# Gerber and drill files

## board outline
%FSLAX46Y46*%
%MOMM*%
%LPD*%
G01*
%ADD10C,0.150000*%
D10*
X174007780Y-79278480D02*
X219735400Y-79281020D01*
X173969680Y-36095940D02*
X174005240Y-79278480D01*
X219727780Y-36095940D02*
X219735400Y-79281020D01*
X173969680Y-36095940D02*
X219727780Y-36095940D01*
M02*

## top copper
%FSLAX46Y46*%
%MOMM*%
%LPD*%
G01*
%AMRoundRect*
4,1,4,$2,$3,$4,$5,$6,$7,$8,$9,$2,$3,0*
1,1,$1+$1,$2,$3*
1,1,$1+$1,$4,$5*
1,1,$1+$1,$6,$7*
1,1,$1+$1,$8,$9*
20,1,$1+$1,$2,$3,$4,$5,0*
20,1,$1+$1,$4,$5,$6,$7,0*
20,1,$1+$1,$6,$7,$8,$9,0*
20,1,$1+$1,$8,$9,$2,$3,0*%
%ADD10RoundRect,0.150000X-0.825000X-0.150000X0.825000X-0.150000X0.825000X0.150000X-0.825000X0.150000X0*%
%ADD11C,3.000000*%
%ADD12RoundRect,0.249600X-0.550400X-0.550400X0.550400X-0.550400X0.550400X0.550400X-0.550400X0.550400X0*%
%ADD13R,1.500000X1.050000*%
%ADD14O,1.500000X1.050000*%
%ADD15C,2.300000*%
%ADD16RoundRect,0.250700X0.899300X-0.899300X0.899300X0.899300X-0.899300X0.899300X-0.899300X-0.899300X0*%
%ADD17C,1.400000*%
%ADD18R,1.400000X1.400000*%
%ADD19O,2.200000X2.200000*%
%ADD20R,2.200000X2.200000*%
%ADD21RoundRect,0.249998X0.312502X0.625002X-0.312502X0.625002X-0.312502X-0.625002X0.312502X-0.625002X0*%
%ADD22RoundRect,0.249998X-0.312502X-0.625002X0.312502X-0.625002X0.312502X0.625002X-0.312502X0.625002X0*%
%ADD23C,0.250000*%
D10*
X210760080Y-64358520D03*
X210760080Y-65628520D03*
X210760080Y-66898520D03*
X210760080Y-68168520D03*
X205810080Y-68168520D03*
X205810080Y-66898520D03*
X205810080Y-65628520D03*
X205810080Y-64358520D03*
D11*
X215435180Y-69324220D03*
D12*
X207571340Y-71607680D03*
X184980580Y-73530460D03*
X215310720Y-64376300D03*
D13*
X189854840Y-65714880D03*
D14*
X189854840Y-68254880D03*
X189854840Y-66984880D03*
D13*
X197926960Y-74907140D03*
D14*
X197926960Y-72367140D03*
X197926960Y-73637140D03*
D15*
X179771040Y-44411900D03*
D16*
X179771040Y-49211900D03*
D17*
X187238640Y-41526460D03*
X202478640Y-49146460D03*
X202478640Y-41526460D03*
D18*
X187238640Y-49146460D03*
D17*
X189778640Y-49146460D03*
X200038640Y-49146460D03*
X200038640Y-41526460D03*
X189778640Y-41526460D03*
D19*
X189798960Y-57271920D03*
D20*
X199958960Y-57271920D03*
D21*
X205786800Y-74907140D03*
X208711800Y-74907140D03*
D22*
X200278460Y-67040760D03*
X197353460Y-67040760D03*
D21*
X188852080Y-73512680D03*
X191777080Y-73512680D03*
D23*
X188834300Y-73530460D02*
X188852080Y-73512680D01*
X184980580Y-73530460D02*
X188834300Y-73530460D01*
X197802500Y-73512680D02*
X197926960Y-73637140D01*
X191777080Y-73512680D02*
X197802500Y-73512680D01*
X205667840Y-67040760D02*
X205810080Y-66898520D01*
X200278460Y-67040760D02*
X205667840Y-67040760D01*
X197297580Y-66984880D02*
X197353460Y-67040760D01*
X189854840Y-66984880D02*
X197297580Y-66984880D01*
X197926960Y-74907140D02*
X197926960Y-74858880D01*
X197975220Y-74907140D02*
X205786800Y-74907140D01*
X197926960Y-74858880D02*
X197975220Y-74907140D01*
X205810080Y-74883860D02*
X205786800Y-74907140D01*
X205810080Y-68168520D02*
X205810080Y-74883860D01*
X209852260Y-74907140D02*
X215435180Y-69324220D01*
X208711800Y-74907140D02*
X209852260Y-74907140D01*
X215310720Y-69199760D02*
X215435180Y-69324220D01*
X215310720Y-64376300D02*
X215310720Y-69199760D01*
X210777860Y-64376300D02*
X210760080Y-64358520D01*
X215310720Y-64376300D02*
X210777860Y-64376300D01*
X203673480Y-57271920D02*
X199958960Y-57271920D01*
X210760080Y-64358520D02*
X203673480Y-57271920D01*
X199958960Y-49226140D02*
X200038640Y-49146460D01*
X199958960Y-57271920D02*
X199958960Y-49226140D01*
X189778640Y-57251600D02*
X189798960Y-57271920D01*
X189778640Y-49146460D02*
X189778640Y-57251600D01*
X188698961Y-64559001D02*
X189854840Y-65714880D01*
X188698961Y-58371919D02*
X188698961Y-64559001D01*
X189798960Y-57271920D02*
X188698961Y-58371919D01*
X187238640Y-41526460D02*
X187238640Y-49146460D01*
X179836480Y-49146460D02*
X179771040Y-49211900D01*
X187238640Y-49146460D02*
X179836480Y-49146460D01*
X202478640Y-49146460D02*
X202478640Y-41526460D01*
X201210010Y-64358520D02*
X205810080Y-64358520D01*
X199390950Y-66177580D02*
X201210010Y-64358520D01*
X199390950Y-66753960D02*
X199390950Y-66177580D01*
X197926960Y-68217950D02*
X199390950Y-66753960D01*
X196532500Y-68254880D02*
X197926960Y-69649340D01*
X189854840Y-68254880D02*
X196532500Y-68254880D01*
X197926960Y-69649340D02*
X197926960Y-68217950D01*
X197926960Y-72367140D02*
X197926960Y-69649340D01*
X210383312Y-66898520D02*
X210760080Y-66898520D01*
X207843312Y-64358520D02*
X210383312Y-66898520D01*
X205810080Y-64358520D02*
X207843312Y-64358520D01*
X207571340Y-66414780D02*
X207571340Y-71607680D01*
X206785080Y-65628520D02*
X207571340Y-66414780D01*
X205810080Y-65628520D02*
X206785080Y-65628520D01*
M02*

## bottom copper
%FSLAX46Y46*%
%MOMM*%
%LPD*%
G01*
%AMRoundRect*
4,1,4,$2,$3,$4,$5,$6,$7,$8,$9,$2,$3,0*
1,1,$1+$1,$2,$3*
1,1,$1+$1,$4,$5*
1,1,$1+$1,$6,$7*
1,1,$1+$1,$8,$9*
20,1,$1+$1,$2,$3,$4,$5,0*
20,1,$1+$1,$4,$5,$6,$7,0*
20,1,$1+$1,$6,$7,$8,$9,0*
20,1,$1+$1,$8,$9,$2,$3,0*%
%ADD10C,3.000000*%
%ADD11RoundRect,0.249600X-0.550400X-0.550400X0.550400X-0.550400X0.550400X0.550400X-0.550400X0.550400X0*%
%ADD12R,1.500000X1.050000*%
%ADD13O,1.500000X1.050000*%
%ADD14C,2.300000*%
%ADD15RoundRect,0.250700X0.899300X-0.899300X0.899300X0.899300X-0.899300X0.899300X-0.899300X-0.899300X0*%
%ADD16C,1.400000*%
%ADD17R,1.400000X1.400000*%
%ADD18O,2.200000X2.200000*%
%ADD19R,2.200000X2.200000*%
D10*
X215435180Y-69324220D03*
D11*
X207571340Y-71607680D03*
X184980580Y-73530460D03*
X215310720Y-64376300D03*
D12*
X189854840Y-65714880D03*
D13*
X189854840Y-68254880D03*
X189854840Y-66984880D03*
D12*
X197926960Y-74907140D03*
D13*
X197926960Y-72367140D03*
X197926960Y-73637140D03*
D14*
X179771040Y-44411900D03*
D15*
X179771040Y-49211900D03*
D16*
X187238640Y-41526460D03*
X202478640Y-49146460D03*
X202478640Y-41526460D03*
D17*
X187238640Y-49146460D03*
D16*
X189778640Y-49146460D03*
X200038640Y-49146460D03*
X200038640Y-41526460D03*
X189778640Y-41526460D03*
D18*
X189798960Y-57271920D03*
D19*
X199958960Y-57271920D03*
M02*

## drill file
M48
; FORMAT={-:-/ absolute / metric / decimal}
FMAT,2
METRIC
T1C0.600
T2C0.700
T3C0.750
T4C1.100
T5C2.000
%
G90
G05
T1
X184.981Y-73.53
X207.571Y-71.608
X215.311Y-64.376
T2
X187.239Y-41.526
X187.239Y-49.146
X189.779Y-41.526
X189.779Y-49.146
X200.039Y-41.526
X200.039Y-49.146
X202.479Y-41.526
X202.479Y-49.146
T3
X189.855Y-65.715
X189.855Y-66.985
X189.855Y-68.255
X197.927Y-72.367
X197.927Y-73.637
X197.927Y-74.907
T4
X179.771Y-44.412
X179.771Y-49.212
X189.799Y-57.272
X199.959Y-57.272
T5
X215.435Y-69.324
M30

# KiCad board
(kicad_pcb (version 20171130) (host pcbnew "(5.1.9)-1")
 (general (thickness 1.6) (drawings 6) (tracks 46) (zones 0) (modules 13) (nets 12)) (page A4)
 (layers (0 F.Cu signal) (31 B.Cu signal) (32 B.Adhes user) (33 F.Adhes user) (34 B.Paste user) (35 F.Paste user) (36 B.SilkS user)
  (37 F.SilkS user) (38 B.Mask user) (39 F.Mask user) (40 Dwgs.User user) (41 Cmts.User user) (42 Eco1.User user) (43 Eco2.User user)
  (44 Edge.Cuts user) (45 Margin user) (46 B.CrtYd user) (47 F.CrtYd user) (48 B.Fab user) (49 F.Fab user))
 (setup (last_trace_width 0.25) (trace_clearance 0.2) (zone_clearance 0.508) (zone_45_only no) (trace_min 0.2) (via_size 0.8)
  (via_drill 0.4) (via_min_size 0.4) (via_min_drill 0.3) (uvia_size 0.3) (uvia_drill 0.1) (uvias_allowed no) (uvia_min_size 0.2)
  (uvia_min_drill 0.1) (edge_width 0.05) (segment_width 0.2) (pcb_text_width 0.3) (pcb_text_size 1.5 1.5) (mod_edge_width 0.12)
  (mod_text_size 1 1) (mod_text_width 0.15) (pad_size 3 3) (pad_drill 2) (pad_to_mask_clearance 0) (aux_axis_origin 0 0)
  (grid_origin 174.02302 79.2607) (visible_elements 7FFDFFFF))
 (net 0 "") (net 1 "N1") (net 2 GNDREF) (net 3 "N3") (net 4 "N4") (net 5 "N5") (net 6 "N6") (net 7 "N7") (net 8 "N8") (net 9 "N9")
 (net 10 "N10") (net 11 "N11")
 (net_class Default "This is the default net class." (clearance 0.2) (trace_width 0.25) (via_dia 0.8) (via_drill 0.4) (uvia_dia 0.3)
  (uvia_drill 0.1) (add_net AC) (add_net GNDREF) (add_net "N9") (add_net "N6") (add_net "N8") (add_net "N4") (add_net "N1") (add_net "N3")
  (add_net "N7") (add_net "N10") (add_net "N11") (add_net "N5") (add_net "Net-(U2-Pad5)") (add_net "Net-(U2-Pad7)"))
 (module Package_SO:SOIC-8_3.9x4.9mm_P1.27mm (layer F.Cu) (at 208.28508 66.26352)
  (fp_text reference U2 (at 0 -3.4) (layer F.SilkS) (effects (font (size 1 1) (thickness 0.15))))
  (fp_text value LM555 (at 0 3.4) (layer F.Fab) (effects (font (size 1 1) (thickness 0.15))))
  (pad 8 smd roundrect (at 2.475 -1.905) (size 1.95 0.6) (layers F.Cu F.Paste F.Mask) (roundrect_rratio 0.25) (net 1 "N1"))
  (pad 7 smd roundrect (at 2.475 -0.635) (size 1.95 0.6) (layers F.Cu F.Paste F.Mask) (roundrect_rratio 0.25))
  (pad 6 smd roundrect (at 2.475 0.635) (size 1.95 0.6) (layers F.Cu F.Paste F.Mask) (roundrect_rratio 0.25) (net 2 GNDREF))
  (pad 5 smd roundrect (at 2.475 1.905) (size 1.95 0.6) (layers F.Cu F.Paste F.Mask) (roundrect_rratio 0.25))
  (pad 4 smd roundrect (at -2.475 1.905) (size 1.95 0.6) (layers F.Cu F.Paste F.Mask) (roundrect_rratio 0.25) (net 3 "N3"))
  (pad 3 smd roundrect (at -2.475 0.635) (size 1.95 0.6) (layers F.Cu F.Paste F.Mask) (roundrect_rratio 0.25) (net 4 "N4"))
  (pad 2 smd roundrect (at -2.475 -0.635) (size 1.95 0.6) (layers F.Cu F.Paste F.Mask) (roundrect_rratio 0.25) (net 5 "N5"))
  (pad 1 smd roundrect (at -2.475 -1.905) (size 1.95 0.6) (layers F.Cu F.Paste F.Mask) (roundrect_rratio 0.25) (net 2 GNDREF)))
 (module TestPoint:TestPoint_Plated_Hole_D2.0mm (layer F.Cu) (at 215.43518 69.32422)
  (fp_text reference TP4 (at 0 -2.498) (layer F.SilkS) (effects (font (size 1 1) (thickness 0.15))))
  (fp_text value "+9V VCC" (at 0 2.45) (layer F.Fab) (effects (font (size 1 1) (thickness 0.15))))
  (pad 1 thru_hole circle (at 0 0) (size 3 3) (drill 2) (layers *.Mask F.Cu) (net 1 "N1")))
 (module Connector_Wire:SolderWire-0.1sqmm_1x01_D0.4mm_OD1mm (layer F.Cu) (at 207.57134 71.60768)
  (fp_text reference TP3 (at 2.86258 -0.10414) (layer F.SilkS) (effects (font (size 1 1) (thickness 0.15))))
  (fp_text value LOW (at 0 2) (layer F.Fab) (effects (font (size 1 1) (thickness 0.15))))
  (pad 1 thru_hole roundrect (at 0 0) (size 1.6 1.6) (drill 0.6) (layers *.Mask F.Cu) (roundrect_rratio 0.156) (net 5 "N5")))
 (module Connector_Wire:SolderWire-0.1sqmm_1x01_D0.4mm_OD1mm (layer F.Cu) (at 184.98058 73.53046)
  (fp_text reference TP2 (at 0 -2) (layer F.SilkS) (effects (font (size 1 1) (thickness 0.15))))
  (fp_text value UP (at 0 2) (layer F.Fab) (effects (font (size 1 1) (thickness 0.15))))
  (pad 1 thru_hole roundrect (at 0 0) (size 1.6 1.6) (drill 0.6) (layers *.Mask F.Cu) (roundrect_rratio 0.156) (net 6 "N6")))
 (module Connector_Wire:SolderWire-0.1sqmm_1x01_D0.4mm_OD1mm (layer F.Cu) (at 215.31072 64.3763)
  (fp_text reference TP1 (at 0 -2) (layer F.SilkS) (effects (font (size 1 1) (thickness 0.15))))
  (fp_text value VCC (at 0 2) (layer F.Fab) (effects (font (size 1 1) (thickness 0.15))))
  (pad 1 thru_hole roundrect (at 0 0) (size 1.6 1.6) (drill 0.6) (layers *.Mask F.Cu) (roundrect_rratio 0.156) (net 1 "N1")))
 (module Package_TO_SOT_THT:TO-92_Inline (layer F.Cu) (at 189.85484 65.71488 270)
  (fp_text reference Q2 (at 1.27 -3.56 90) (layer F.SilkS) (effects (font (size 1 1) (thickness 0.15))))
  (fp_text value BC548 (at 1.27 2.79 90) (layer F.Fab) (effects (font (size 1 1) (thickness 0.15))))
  (pad 1 thru_hole rect (at 0 0 270) (size 1.05 1.5) (drill 0.75) (layers *.Mask F.Cu) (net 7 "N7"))
  (pad 3 thru_hole oval (at 2.54 0 270) (size 1.05 1.5) (drill 0.75) (layers *.Mask F.Cu) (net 2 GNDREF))
  (pad 2 thru_hole oval (at 1.27 0 270) (size 1.05 1.5) (drill 0.75) (layers *.Mask F.Cu) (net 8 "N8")))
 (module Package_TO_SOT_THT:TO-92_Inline (layer F.Cu) (at 197.92696 74.90714 90)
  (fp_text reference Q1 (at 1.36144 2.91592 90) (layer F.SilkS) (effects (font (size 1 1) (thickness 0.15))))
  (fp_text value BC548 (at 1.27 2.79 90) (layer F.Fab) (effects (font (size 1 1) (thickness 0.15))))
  (pad 1 thru_hole rect (at 0 0 90) (size 1.05 1.5) (drill 0.75) (layers *.Mask F.Cu) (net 3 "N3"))
  (pad 3 thru_hole oval (at 2.54 0 90) (size 1.05 1.5) (drill 0.75) (layers *.Mask F.Cu) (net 2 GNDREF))
  (pad 2 thru_hole oval (at 1.27 0 90) (size 1.05 1.5) (drill 0.75) (layers *.Mask F.Cu) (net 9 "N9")))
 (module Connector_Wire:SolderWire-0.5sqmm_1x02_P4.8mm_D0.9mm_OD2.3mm (layer F.Cu) (at 179.77104 49.2119 90)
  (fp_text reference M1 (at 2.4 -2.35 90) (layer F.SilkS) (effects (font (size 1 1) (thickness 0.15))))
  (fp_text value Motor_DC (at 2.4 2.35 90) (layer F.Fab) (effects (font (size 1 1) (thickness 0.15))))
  (pad 2 thru_hole circle (at 4.8 0 90) (size 2.3 2.3) (drill 1.1) (layers *.Mask F.Cu))
  (pad 1 thru_hole roundrect (at 0 0 90) (size 2.3 2.3) (drill 1.1) (layers *.Mask F.Cu) (roundrect_rratio 0.109) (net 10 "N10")))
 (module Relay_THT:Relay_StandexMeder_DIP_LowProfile (layer F.Cu) (at 187.23864 49.14646 90)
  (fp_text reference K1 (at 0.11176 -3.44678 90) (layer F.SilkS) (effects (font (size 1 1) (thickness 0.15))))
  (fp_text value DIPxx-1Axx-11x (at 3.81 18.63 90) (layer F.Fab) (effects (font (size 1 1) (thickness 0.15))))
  (pad 14 thru_hole circle (at 7.62 0 90) (size 1.4 1.4) (drill 0.7) (layers *.Mask F.Cu) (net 10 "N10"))
  (pad 7 thru_hole circle (at 0 15.24 90) (size 1.4 1.4) (drill 0.7) (layers *.Mask F.Cu) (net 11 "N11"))
  (pad 8 thru_hole circle (at 7.62 15.24 90) (size 1.4 1.4) (drill 0.7) (layers *.Mask F.Cu) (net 11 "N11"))
  (pad 1 thru_hole rect (at 0 0 90) (size 1.4 1.4) (drill 0.7) (layers *.Mask F.Cu) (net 10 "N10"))
  (pad 2 thru_hole circle (at 0 2.54 90) (size 1.4 1.4) (drill 0.7) (layers *.Mask F.Cu) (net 7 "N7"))
  (pad 6 thru_hole circle (at 0 12.8 90) (size 1.4 1.4) (drill 0.7) (layers *.Mask F.Cu) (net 1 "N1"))
  (pad 9 thru_hole circle (at 7.62 12.8 90) (size 1.4 1.4) (drill 0.7) (layers *.Mask F.Cu))
  (pad 13 thru_hole circle (at 7.62 2.54 90) (size 1.4 1.4) (drill 0.7) (layers *.Mask F.Cu)))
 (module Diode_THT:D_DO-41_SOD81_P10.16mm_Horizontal (layer F.Cu) (at 199.95896 57.27192 180)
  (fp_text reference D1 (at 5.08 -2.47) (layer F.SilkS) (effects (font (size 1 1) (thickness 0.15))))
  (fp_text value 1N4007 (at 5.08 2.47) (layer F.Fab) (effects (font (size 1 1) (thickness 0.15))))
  (pad 2 thru_hole oval (at 10.16 0 180) (size 2.2 2.2) (drill 1.1) (layers *.Mask F.Cu) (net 7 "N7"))
  (pad 1 thru_hole rect (at 0 0 180) (size 2.2 2.2) (drill 1.1) (layers *.Mask F.Cu) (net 1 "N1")))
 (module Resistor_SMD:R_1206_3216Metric (layer F.Cu) (at 207.2493 74.90714 180)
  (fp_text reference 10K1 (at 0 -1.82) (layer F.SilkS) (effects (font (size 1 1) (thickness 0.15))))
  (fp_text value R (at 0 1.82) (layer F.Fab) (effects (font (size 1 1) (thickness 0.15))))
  (pad 2 smd roundrect (at 1.4625 0 180) (size 1.125 1.75) (layers F.Cu F.Paste F.Mask) (roundrect_rratio 0.2222204444444444) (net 3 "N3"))
  (pad 1 smd roundrect (at -1.4625 0 180) (size 1.125 1.75) (layers F.Cu F.Paste F.Mask) (roundrect_rratio 0.2222204444444444) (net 1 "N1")))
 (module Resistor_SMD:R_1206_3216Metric (layer F.Cu) (at 198.81596 67.04076)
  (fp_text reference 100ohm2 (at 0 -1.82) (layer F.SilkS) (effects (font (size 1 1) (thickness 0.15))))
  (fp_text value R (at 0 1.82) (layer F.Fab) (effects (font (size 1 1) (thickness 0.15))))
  (pad 2 smd roundrect (at 1.4625 0) (size 1.125 1.75) (layers F.Cu F.Paste F.Mask) (roundrect_rratio 0.2222204444444444) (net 4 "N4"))
  (pad 1 smd roundrect (at -1.4625 0) (size 1.125 1.75) (layers F.Cu F.Paste F.Mask) (roundrect_rratio 0.2222204444444444) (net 8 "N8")))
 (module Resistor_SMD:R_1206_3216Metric (layer F.Cu) (at 190.31458 73.51268 180)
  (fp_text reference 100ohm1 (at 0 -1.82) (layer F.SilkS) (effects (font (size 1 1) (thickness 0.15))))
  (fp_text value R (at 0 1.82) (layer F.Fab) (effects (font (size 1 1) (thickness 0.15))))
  (pad 2 smd roundrect (at 1.4625 0 180) (size 1.125 1.75) (layers F.Cu F.Paste F.Mask) (roundrect_rratio 0.2222204444444444) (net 6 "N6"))
  (pad 1 smd roundrect (at -1.4625 0 180) (size 1.125 1.75) (layers F.Cu F.Paste F.Mask) (roundrect_rratio 0.2222204444444444) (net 9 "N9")))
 (gr_line (start 174.00778 79.27848) (end 219.7354 79.28102) (layer Edge.Cuts) (width 0.15))
 (gr_line (start 173.96968 36.09594) (end 174.00524 79.27848) (layer Edge.Cuts) (width 0.15))
 (gr_line (start 219.72778 36.09594) (end 219.7354 79.28102) (layer Edge.Cuts) (width 0.15))
 (gr_line (start 173.96968 36.09594) (end 219.72778 36.09594) (layer Edge.Cuts) (width 0.15))
 (segment (start 188.8343 73.53046) (end 188.85208 73.51268) (width 0.25) (layer F.Cu) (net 6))
 (segment (start 184.98058 73.53046) (end 188.8343 73.53046) (width 0.25) (layer F.Cu) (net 6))
 (segment (start 197.8025 73.51268) (end 197.92696 73.63714) (width 0.25) (layer F.Cu) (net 9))
 (segment (start 191.77708 73.51268) (end 197.8025 73.51268) (width 0.25) (layer F.Cu) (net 9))
 (segment (start 205.66784 67.04076) (end 205.81008 66.89852) (width 0.25) (layer F.Cu) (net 4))
 (segment (start 200.27846 67.04076) (end 205.66784 67.04076) (width 0.25) (layer F.Cu) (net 4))
 (segment (start 197.29758 66.98488) (end 197.35346 67.04076) (width 0.25) (layer F.Cu) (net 8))
 (segment (start 189.85484 66.98488) (end 197.29758 66.98488) (width 0.25) (layer F.Cu) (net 8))
 (segment (start 197.92696 74.90714) (end 197.92696 74.85888) (width 0.25) (layer F.Cu) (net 3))
 (segment (start 197.97522 74.90714) (end 205.7868 74.90714) (width 0.25) (layer F.Cu) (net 3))
 (segment (start 197.92696 74.85888) (end 197.97522 74.90714) (width 0.25) (layer F.Cu) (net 3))
 (segment (start 205.81008 74.88386) (end 205.7868 74.90714) (width 0.25) (layer F.Cu) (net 3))
 (segment (start 205.81008 68.16852) (end 205.81008 74.88386) (width 0.25) (layer F.Cu) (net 3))
 (segment (start 209.85226 74.90714) (end 215.43518 69.32422) (width 0.25) (layer F.Cu) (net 1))
 (segment (start 208.7118 74.90714) (end 209.85226 74.90714) (width 0.25) (layer F.Cu) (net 1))
 (segment (start 215.31072 69.19976) (end 215.43518 69.32422) (width 0.25) (layer F.Cu) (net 1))
 (segment (start 215.31072 64.3763) (end 215.31072 69.19976) (width 0.25) (layer F.Cu) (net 1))
 (segment (start 210.77786 64.3763) (end 210.76008 64.35852) (width 0.25) (layer F.Cu) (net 1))
 (segment (start 215.31072 64.3763) (end 210.77786 64.3763) (width 0.25) (layer F.Cu) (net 1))
 (segment (start 203.67348 57.27192) (end 199.95896 57.27192) (width 0.25) (layer F.Cu) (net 1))
 (segment (start 210.76008 64.35852) (end 203.67348 57.27192) (width 0.25) (layer F.Cu) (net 1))
 (segment (start 199.95896 49.22614) (end 200.03864 49.14646) (width 0.25) (layer F.Cu) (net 1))
 (segment (start 199.95896 57.27192) (end 199.95896 49.22614) (width 0.25) (layer F.Cu) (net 1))
 (segment (start 189.77864 57.2516) (end 189.79896 57.27192) (width 0.25) (layer F.Cu) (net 7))
 (segment (start 189.77864 49.14646) (end 189.77864 57.2516) (width 0.25) (layer F.Cu) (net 7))
 (segment (start 188.698961 64.559001) (end 189.85484 65.71488) (width 0.25) (layer F.Cu) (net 7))
 (segment (start 188.698961 58.371919) (end 188.698961 64.559001) (width 0.25) (layer F.Cu) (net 7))
 (segment (start 189.79896 57.27192) (end 188.698961 58.371919) (width 0.25) (layer F.Cu) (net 7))
 (segment (start 187.23864 41.52646) (end 187.23864 49.14646) (width 0.25) (layer F.Cu) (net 10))
 (segment (start 179.83648 49.14646) (end 179.77104 49.2119) (width 0.25) (layer F.Cu) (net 10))
 (segment (start 187.23864 49.14646) (end 179.83648 49.14646) (width 0.25) (layer F.Cu) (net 10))
 (segment (start 202.47864 49.14646) (end 202.47864 41.52646) (width 0.25) (layer F.Cu) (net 11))
 (segment (start 201.21001 64.35852) (end 205.81008 64.35852) (width 0.25) (layer F.Cu) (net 2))
 (segment (start 199.39095 66.17758) (end 201.21001 64.35852) (width 0.25) (layer F.Cu) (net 2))
 (segment (start 199.39095 66.75396) (end 199.39095 66.17758) (width 0.25) (layer F.Cu) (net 2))
 (segment (start 197.92696 68.21795) (end 199.39095 66.75396) (width 0.25) (layer F.Cu) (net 2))
 (segment (start 196.5325 68.25488) (end 197.92696 69.64934) (width 0.25) (layer F.Cu) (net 2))
 (segment (start 189.85484 68.25488) (end 196.5325 68.25488) (width 0.25) (layer F.Cu) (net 2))
 (segment (start 197.92696 69.64934) (end 197.92696 68.21795) (width 0.25) (layer F.Cu) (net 2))
 (segment (start 197.92696 72.36714) (end 197.92696 69.64934) (width 0.25) (layer F.Cu) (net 2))
 (segment (start 210.383312 66.89852) (end 210.76008 66.89852) (width 0.25) (layer F.Cu) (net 2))
 (segment (start 207.843312 64.35852) (end 210.383312 66.89852) (width 0.25) (layer F.Cu) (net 2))
 (segment (start 205.81008 64.35852) (end 207.843312 64.35852) (width 0.25) (layer F.Cu) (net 2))
 (segment (start 207.57134 66.41478) (end 207.57134 71.60768) (width 0.25) (layer F.Cu) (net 5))
 (segment (start 206.78508 65.62852) (end 207.57134 66.41478) (width 0.25) (layer F.Cu) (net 5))
 (segment (start 205.81008 65.62852) (end 206.78508 65.62852) (width 0.25) (layer F.Cu) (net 5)))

